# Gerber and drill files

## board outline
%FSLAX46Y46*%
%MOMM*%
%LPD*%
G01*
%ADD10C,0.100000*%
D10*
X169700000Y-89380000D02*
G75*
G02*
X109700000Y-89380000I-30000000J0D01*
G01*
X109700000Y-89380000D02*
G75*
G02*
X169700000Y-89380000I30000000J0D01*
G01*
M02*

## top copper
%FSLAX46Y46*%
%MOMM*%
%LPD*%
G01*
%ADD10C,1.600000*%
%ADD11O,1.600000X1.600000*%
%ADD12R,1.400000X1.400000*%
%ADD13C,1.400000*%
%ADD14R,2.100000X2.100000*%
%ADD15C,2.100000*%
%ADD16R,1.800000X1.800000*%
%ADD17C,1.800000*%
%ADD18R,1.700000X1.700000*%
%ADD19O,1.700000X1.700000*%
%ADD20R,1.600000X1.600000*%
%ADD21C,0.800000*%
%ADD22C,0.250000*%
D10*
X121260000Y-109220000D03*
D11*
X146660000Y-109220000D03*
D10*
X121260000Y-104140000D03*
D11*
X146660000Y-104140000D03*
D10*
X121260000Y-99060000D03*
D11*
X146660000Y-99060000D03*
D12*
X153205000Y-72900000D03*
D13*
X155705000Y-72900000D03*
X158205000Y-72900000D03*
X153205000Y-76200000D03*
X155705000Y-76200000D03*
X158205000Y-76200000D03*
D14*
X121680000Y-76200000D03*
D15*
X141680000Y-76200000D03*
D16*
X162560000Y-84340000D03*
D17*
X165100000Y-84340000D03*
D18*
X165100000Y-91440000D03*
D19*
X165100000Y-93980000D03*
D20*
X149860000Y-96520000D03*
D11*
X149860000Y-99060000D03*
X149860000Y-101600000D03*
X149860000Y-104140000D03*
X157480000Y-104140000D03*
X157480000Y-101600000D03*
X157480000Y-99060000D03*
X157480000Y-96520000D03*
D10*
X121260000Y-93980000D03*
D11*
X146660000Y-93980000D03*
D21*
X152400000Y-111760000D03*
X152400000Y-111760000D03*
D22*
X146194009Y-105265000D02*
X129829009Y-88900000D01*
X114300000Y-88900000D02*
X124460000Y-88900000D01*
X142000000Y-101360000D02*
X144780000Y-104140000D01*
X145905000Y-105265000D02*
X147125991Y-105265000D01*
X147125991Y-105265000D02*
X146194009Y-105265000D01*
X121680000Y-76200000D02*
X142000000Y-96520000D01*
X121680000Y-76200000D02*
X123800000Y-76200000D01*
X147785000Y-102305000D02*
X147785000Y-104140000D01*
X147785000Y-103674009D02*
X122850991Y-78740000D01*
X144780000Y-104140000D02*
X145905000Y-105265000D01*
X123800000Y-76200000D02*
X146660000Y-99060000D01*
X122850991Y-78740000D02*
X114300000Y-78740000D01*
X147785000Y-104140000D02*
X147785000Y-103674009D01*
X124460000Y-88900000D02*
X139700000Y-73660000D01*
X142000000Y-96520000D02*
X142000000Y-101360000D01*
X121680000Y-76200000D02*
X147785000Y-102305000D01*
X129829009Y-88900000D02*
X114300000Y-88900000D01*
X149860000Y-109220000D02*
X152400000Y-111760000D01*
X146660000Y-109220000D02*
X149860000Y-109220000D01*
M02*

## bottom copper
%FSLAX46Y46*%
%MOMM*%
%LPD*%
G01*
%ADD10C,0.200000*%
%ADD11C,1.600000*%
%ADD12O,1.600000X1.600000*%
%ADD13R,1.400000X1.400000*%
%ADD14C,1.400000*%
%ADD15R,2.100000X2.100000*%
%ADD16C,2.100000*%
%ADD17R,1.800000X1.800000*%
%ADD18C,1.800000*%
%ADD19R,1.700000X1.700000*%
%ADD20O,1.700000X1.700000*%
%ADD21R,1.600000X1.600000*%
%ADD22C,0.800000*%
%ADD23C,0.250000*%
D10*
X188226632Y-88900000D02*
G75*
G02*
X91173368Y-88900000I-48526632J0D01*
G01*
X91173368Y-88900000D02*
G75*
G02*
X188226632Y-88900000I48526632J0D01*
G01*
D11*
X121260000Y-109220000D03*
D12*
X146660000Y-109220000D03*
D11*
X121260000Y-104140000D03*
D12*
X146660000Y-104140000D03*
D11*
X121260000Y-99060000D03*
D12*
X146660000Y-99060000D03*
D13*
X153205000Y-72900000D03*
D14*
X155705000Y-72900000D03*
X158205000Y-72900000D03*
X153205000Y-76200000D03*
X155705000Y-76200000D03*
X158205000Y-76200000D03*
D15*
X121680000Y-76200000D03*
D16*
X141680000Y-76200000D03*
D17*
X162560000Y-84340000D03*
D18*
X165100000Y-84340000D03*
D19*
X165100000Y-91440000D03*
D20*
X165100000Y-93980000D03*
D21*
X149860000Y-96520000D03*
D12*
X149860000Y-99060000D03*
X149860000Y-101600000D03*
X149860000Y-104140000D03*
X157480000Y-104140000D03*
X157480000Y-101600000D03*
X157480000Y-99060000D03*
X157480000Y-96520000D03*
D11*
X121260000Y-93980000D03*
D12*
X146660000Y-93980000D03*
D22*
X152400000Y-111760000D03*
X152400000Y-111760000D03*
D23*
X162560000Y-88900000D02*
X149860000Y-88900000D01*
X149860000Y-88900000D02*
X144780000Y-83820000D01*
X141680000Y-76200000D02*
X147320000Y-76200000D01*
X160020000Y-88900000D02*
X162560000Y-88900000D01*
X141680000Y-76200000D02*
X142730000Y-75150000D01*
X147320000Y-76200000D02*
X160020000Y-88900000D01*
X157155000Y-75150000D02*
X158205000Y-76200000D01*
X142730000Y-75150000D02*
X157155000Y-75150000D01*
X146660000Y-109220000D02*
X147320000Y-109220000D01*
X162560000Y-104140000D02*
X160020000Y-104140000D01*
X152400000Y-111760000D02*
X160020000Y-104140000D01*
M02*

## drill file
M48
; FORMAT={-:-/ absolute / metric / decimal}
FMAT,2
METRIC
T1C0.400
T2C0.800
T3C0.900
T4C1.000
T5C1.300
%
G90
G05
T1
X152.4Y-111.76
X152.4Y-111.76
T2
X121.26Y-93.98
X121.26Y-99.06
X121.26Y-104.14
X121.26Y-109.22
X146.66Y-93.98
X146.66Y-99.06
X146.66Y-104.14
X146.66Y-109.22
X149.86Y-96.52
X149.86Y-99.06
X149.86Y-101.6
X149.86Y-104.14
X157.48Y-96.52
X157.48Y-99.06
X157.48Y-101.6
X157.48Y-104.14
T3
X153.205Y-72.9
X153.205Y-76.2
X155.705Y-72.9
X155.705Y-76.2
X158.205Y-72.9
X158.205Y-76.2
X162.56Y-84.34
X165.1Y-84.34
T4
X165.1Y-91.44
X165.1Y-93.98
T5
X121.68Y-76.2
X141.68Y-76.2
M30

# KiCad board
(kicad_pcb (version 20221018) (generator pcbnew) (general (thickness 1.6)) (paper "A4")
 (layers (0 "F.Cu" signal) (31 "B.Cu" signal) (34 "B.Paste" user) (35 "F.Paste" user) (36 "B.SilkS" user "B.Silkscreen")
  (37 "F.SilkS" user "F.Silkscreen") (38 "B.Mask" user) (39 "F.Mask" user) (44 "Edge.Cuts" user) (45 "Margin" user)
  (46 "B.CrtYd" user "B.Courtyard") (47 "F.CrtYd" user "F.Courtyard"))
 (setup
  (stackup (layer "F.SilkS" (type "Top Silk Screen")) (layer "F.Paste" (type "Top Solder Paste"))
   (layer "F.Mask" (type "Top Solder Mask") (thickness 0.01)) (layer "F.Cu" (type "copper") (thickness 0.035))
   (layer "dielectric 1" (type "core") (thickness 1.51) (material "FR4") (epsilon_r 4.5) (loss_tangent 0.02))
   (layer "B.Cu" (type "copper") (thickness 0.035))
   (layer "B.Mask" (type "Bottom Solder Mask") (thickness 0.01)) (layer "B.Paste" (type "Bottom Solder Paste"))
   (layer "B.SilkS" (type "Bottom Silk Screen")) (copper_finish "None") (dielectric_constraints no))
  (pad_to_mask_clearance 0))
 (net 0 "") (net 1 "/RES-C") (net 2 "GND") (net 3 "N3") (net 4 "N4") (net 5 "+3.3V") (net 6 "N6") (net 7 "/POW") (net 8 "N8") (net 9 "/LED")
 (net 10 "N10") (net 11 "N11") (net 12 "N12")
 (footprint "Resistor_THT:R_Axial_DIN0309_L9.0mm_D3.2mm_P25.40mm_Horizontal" (layer "F.Cu") (at 121.26 109.22)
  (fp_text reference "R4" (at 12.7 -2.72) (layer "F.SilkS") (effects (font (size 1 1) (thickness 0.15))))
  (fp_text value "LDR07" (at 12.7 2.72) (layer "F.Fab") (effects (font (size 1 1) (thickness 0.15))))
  (pad "1" thru_hole circle (at 0 0) (size 1.6 1.6) (drill 0.8) (layers "*.Cu" "*.Mask") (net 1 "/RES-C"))
  (pad "2" thru_hole oval (at 25.4 0) (size 1.6 1.6) (drill 0.8) (layers "*.Cu" "*.Mask") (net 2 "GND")))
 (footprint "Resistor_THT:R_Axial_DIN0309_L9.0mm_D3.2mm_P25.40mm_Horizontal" (layer "F.Cu") (at 121.26 104.14)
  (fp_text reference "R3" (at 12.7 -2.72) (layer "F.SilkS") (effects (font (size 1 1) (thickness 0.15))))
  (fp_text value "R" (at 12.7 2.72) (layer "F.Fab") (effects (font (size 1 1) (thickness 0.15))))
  (pad "1" thru_hole circle (at 0 0) (size 1.6 1.6) (drill 0.8) (layers "*.Cu" "*.Mask") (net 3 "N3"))
  (pad "2" thru_hole oval (at 25.4 0) (size 1.6 1.6) (drill 0.8) (layers "*.Cu" "*.Mask") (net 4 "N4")))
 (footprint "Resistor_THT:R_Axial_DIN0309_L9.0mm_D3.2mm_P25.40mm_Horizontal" (layer "F.Cu") (at 121.26 99.06)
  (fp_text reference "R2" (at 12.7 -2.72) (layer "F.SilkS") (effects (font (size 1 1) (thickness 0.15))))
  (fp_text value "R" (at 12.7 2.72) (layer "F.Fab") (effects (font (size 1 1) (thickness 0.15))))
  (pad "1" thru_hole circle (at 0 0) (size 1.6 1.6) (drill 0.8) (layers "*.Cu" "*.Mask") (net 1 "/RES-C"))
  (pad "2" thru_hole oval (at 25.4 0) (size 1.6 1.6) (drill 0.8) (layers "*.Cu" "*.Mask") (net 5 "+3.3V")))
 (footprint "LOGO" (layer "F.Cu") (at 152.4 88.9)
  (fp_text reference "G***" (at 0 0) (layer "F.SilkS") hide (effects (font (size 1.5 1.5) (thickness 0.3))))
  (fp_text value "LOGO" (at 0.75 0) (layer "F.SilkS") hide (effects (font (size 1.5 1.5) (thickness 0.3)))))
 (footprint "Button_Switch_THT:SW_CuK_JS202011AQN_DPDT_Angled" (layer "F.Cu") (at 153.205 72.9)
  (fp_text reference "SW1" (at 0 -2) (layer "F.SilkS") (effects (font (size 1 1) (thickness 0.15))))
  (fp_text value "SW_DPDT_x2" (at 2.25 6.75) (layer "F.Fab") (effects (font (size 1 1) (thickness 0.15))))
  (pad "1" thru_hole rect (at 0 0) (size 1.4 1.4) (drill 0.9) (layers "*.Cu" "*.Mask"))
  (pad "2" thru_hole circle (at 2.5 0) (size 1.4 1.4) (drill 0.9) (layers "*.Cu" "*.Mask"))
  (pad "3" thru_hole circle (at 5 0) (size 1.4 1.4) (drill 0.9) (layers "*.Cu" "*.Mask"))
  (pad "4" thru_hole circle (at 0 3.3) (size 1.4 1.4) (drill 0.9) (layers "*.Cu" "*.Mask") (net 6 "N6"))
  (pad "5" thru_hole circle (at 2.5 3.3) (size 1.4 1.4) (drill 0.9) (layers "*.Cu" "*.Mask") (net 2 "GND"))
  (pad "6" thru_hole circle (at 5 3.3) (size 1.4 1.4) (drill 0.9) (layers "*.Cu" "*.Mask") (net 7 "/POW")))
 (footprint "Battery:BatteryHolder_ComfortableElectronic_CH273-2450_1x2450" (layer "F.Cu") (at 121.68 76.2)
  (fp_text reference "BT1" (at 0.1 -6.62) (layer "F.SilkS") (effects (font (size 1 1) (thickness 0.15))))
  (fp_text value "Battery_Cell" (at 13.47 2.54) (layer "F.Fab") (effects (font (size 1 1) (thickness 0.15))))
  (pad "1" thru_hole rect (at 0 0 270) (size 2.1 2.1) (drill 1.3) (layers "*.Cu" "*.Mask") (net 5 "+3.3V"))
  (pad "2" thru_hole circle (at 20 0 270) (size 2.1 2.1) (drill 1.3) (layers "*.Cu" "*.Mask") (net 7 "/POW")))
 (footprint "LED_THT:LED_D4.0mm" (layer "F.Cu") (at 162.56 84.34)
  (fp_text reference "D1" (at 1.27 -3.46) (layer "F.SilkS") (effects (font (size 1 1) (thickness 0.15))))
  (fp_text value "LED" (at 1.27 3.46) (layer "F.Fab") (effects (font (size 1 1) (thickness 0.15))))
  (pad "1" thru_hole rect (at 0 0) (size 1.8 1.8) (drill 0.9) (layers "*.Cu" "*.Mask") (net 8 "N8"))
  (pad "2" thru_hole circle (at 2.54 0) (size 1.8 1.8) (drill 0.9) (layers "*.Cu" "*.Mask") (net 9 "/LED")))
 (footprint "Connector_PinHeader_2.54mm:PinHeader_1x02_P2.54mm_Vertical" (layer "F.Cu") (at 165.1 91.44)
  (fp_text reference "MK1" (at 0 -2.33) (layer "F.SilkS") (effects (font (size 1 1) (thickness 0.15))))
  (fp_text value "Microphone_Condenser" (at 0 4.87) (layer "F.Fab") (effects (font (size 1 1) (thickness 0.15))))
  (pad "1" thru_hole rect (at 0 0) (size 1.7 1.7) (drill 1) (layers "*.Cu" "*.Mask") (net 2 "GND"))
  (pad "2" thru_hole oval (at 0 2.54) (size 1.7 1.7) (drill 1) (layers "*.Cu" "*.Mask") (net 4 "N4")))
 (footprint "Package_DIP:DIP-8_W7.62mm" (layer "F.Cu") (at 149.86 96.52)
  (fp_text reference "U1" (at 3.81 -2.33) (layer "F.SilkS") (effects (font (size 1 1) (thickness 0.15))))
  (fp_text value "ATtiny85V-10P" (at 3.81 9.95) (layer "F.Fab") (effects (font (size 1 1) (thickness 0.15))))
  (pad "1" thru_hole rect (at 0 0) (size 1.6 1.6) (drill 0.8) (layers "*.Cu" "*.Mask") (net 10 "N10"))
  (pad "2" thru_hole oval (at 0 2.54) (size 1.6 1.6) (drill 0.8) (layers "*.Cu" "*.Mask") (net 1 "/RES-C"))
  (pad "3" thru_hole oval (at 0 5.08) (size 1.6 1.6) (drill 0.8) (layers "*.Cu" "*.Mask") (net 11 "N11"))
  (pad "4" thru_hole oval (at 0 7.62) (size 1.6 1.6) (drill 0.8) (layers "*.Cu" "*.Mask") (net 2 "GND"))
  (pad "5" thru_hole oval (at 7.62 7.62) (size 1.6 1.6) (drill 0.8) (layers "*.Cu" "*.Mask") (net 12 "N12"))
  (pad "6" thru_hole oval (at 7.62 5.08) (size 1.6 1.6) (drill 0.8) (layers "*.Cu" "*.Mask") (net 9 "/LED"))
  (pad "7" thru_hole oval (at 7.62 2.54) (size 1.6 1.6) (drill 0.8) (layers "*.Cu" "*.Mask") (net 3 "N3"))
  (pad "8" thru_hole oval (at 7.62 0) (size 1.6 1.6) (drill 0.8) (layers "*.Cu" "*.Mask") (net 5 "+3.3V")))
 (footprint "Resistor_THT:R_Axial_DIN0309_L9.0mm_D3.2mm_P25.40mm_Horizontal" (layer "F.Cu") (at 121.26 93.98)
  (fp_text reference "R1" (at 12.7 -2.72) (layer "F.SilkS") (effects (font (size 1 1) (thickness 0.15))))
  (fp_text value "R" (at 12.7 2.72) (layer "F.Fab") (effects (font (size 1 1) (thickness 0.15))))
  (pad "1" thru_hole circle (at 0 0) (size 1.6 1.6) (drill 0.8) (layers "*.Cu" "*.Mask") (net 8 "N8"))
  (pad "2" thru_hole oval (at 25.4 0) (size 1.6 1.6) (drill 0.8) (layers "*.Cu" "*.Mask") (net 2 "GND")))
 (gr_circle (center 139.7 88.9) (end 104.14 121.92) (stroke (width 0.2) (type default)) (fill none) (layer "B.Cu"))
 (gr_circle locked (center 139.7 89.38) (end 169.7 89.38) (stroke (width 0.1) (type default)) (fill none) (layer "Edge.Cuts"))
 (segment (start 146.194009 105.265) (end 129.829009 88.9) (width 0.25) (layer "F.Cu") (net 5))
 (segment (start 114.3 88.9) (end 124.46 88.9) (width 0.25) (layer "F.Cu") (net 5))
 (segment (start 142 101.36) (end 144.78 104.14) (width 0.25) (layer "F.Cu") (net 5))
 (segment (start 145.905 105.265) (end 147.125991 105.265) (width 0.25) (layer "F.Cu") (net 5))
 (segment (start 147.125991 105.265) (end 146.194009 105.265) (width 0.25) (layer "F.Cu") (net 5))
 (segment (start 121.68 76.2) (end 142 96.52) (width 0.25) (layer "F.Cu") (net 5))
 (segment (start 121.68 76.2) (end 123.8 76.2) (width 0.25) (layer "F.Cu") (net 5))
 (segment (start 147.785 102.305) (end 147.785 104.14) (width 0.25) (layer "F.Cu") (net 5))
 (segment (start 147.785 103.674009) (end 122.850991 78.74) (width 0.25) (layer "F.Cu") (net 5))
 (segment (start 144.78 104.14) (end 145.905 105.265) (width 0.25) (layer "F.Cu") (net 5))
 (segment (start 123.8 76.2) (end 146.66 99.06) (width 0.25) (layer "F.Cu") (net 5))
 (segment (start 122.850991 78.74) (end 114.3 78.74) (width 0.25) (layer "F.Cu") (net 5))
 (segment (start 147.785 104.14) (end 147.785 103.674009) (width 0.25) (layer "F.Cu") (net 5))
 (segment (start 124.46 88.9) (end 139.7 73.66) (width 0.25) (layer "F.Cu") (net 5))
 (segment (start 142 96.52) (end 142 101.36) (width 0.25) (layer "F.Cu") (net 5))
 (segment (start 121.68 76.2) (end 147.785 102.305) (width 0.25) (layer "F.Cu") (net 5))
 (segment (start 129.829009 88.9) (end 114.3 88.9) (width 0.25) (layer "F.Cu") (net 5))
 (segment (start 162.56 88.9) (end 149.86 88.9) (width 0.25) (layer "B.Cu") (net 7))
 (segment (start 149.86 88.9) (end 144.78 83.82) (width 0.25) (layer "B.Cu") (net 7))
 (segment (start 141.68 76.2) (end 147.32 76.2) (width 0.25) (layer "B.Cu") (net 7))
 (segment (start 160.02 88.9) (end 162.56 88.9) (width 0.25) (layer "B.Cu") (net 7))
 (segment (start 141.68 76.2) (end 142.73 75.15) (width 0.25) (layer "B.Cu") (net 7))
 (segment (start 147.32 76.2) (end 160.02 88.9) (width 0.25) (layer "B.Cu") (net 7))
 (segment (start 157.155 75.15) (end 158.205 76.2) (width 0.25) (layer "B.Cu") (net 7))
 (segment (start 142.73 75.15) (end 157.155 75.15) (width 0.25) (layer "B.Cu") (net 7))
 (segment (start 149.86 109.22) (end 152.4 111.76) (width 0.25) (layer "F.Cu") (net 2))
 (segment (start 146.66 109.22) (end 149.86 109.22) (width 0.25) (layer "F.Cu") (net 2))
 (via (at 152.4 111.76) (size 0.8) (drill 0.4) (layers "F.Cu" "B.Cu") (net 2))
 (via (at 152.4 111.76) (size 0.8) (drill 0.4) (layers "F.Cu" "B.Cu") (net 2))
 (segment (start 146.66 109.22) (end 147.32 109.22) (width 0.25) (layer "B.Cu") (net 2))
 (segment (start 162.56 104.14) (end 160.02 104.14) (width 0.25) (layer "B.Cu") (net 2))
 (segment (start 152.4 111.76) (end 160.02 104.14) (width 0.25) (layer "B.Cu") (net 2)))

